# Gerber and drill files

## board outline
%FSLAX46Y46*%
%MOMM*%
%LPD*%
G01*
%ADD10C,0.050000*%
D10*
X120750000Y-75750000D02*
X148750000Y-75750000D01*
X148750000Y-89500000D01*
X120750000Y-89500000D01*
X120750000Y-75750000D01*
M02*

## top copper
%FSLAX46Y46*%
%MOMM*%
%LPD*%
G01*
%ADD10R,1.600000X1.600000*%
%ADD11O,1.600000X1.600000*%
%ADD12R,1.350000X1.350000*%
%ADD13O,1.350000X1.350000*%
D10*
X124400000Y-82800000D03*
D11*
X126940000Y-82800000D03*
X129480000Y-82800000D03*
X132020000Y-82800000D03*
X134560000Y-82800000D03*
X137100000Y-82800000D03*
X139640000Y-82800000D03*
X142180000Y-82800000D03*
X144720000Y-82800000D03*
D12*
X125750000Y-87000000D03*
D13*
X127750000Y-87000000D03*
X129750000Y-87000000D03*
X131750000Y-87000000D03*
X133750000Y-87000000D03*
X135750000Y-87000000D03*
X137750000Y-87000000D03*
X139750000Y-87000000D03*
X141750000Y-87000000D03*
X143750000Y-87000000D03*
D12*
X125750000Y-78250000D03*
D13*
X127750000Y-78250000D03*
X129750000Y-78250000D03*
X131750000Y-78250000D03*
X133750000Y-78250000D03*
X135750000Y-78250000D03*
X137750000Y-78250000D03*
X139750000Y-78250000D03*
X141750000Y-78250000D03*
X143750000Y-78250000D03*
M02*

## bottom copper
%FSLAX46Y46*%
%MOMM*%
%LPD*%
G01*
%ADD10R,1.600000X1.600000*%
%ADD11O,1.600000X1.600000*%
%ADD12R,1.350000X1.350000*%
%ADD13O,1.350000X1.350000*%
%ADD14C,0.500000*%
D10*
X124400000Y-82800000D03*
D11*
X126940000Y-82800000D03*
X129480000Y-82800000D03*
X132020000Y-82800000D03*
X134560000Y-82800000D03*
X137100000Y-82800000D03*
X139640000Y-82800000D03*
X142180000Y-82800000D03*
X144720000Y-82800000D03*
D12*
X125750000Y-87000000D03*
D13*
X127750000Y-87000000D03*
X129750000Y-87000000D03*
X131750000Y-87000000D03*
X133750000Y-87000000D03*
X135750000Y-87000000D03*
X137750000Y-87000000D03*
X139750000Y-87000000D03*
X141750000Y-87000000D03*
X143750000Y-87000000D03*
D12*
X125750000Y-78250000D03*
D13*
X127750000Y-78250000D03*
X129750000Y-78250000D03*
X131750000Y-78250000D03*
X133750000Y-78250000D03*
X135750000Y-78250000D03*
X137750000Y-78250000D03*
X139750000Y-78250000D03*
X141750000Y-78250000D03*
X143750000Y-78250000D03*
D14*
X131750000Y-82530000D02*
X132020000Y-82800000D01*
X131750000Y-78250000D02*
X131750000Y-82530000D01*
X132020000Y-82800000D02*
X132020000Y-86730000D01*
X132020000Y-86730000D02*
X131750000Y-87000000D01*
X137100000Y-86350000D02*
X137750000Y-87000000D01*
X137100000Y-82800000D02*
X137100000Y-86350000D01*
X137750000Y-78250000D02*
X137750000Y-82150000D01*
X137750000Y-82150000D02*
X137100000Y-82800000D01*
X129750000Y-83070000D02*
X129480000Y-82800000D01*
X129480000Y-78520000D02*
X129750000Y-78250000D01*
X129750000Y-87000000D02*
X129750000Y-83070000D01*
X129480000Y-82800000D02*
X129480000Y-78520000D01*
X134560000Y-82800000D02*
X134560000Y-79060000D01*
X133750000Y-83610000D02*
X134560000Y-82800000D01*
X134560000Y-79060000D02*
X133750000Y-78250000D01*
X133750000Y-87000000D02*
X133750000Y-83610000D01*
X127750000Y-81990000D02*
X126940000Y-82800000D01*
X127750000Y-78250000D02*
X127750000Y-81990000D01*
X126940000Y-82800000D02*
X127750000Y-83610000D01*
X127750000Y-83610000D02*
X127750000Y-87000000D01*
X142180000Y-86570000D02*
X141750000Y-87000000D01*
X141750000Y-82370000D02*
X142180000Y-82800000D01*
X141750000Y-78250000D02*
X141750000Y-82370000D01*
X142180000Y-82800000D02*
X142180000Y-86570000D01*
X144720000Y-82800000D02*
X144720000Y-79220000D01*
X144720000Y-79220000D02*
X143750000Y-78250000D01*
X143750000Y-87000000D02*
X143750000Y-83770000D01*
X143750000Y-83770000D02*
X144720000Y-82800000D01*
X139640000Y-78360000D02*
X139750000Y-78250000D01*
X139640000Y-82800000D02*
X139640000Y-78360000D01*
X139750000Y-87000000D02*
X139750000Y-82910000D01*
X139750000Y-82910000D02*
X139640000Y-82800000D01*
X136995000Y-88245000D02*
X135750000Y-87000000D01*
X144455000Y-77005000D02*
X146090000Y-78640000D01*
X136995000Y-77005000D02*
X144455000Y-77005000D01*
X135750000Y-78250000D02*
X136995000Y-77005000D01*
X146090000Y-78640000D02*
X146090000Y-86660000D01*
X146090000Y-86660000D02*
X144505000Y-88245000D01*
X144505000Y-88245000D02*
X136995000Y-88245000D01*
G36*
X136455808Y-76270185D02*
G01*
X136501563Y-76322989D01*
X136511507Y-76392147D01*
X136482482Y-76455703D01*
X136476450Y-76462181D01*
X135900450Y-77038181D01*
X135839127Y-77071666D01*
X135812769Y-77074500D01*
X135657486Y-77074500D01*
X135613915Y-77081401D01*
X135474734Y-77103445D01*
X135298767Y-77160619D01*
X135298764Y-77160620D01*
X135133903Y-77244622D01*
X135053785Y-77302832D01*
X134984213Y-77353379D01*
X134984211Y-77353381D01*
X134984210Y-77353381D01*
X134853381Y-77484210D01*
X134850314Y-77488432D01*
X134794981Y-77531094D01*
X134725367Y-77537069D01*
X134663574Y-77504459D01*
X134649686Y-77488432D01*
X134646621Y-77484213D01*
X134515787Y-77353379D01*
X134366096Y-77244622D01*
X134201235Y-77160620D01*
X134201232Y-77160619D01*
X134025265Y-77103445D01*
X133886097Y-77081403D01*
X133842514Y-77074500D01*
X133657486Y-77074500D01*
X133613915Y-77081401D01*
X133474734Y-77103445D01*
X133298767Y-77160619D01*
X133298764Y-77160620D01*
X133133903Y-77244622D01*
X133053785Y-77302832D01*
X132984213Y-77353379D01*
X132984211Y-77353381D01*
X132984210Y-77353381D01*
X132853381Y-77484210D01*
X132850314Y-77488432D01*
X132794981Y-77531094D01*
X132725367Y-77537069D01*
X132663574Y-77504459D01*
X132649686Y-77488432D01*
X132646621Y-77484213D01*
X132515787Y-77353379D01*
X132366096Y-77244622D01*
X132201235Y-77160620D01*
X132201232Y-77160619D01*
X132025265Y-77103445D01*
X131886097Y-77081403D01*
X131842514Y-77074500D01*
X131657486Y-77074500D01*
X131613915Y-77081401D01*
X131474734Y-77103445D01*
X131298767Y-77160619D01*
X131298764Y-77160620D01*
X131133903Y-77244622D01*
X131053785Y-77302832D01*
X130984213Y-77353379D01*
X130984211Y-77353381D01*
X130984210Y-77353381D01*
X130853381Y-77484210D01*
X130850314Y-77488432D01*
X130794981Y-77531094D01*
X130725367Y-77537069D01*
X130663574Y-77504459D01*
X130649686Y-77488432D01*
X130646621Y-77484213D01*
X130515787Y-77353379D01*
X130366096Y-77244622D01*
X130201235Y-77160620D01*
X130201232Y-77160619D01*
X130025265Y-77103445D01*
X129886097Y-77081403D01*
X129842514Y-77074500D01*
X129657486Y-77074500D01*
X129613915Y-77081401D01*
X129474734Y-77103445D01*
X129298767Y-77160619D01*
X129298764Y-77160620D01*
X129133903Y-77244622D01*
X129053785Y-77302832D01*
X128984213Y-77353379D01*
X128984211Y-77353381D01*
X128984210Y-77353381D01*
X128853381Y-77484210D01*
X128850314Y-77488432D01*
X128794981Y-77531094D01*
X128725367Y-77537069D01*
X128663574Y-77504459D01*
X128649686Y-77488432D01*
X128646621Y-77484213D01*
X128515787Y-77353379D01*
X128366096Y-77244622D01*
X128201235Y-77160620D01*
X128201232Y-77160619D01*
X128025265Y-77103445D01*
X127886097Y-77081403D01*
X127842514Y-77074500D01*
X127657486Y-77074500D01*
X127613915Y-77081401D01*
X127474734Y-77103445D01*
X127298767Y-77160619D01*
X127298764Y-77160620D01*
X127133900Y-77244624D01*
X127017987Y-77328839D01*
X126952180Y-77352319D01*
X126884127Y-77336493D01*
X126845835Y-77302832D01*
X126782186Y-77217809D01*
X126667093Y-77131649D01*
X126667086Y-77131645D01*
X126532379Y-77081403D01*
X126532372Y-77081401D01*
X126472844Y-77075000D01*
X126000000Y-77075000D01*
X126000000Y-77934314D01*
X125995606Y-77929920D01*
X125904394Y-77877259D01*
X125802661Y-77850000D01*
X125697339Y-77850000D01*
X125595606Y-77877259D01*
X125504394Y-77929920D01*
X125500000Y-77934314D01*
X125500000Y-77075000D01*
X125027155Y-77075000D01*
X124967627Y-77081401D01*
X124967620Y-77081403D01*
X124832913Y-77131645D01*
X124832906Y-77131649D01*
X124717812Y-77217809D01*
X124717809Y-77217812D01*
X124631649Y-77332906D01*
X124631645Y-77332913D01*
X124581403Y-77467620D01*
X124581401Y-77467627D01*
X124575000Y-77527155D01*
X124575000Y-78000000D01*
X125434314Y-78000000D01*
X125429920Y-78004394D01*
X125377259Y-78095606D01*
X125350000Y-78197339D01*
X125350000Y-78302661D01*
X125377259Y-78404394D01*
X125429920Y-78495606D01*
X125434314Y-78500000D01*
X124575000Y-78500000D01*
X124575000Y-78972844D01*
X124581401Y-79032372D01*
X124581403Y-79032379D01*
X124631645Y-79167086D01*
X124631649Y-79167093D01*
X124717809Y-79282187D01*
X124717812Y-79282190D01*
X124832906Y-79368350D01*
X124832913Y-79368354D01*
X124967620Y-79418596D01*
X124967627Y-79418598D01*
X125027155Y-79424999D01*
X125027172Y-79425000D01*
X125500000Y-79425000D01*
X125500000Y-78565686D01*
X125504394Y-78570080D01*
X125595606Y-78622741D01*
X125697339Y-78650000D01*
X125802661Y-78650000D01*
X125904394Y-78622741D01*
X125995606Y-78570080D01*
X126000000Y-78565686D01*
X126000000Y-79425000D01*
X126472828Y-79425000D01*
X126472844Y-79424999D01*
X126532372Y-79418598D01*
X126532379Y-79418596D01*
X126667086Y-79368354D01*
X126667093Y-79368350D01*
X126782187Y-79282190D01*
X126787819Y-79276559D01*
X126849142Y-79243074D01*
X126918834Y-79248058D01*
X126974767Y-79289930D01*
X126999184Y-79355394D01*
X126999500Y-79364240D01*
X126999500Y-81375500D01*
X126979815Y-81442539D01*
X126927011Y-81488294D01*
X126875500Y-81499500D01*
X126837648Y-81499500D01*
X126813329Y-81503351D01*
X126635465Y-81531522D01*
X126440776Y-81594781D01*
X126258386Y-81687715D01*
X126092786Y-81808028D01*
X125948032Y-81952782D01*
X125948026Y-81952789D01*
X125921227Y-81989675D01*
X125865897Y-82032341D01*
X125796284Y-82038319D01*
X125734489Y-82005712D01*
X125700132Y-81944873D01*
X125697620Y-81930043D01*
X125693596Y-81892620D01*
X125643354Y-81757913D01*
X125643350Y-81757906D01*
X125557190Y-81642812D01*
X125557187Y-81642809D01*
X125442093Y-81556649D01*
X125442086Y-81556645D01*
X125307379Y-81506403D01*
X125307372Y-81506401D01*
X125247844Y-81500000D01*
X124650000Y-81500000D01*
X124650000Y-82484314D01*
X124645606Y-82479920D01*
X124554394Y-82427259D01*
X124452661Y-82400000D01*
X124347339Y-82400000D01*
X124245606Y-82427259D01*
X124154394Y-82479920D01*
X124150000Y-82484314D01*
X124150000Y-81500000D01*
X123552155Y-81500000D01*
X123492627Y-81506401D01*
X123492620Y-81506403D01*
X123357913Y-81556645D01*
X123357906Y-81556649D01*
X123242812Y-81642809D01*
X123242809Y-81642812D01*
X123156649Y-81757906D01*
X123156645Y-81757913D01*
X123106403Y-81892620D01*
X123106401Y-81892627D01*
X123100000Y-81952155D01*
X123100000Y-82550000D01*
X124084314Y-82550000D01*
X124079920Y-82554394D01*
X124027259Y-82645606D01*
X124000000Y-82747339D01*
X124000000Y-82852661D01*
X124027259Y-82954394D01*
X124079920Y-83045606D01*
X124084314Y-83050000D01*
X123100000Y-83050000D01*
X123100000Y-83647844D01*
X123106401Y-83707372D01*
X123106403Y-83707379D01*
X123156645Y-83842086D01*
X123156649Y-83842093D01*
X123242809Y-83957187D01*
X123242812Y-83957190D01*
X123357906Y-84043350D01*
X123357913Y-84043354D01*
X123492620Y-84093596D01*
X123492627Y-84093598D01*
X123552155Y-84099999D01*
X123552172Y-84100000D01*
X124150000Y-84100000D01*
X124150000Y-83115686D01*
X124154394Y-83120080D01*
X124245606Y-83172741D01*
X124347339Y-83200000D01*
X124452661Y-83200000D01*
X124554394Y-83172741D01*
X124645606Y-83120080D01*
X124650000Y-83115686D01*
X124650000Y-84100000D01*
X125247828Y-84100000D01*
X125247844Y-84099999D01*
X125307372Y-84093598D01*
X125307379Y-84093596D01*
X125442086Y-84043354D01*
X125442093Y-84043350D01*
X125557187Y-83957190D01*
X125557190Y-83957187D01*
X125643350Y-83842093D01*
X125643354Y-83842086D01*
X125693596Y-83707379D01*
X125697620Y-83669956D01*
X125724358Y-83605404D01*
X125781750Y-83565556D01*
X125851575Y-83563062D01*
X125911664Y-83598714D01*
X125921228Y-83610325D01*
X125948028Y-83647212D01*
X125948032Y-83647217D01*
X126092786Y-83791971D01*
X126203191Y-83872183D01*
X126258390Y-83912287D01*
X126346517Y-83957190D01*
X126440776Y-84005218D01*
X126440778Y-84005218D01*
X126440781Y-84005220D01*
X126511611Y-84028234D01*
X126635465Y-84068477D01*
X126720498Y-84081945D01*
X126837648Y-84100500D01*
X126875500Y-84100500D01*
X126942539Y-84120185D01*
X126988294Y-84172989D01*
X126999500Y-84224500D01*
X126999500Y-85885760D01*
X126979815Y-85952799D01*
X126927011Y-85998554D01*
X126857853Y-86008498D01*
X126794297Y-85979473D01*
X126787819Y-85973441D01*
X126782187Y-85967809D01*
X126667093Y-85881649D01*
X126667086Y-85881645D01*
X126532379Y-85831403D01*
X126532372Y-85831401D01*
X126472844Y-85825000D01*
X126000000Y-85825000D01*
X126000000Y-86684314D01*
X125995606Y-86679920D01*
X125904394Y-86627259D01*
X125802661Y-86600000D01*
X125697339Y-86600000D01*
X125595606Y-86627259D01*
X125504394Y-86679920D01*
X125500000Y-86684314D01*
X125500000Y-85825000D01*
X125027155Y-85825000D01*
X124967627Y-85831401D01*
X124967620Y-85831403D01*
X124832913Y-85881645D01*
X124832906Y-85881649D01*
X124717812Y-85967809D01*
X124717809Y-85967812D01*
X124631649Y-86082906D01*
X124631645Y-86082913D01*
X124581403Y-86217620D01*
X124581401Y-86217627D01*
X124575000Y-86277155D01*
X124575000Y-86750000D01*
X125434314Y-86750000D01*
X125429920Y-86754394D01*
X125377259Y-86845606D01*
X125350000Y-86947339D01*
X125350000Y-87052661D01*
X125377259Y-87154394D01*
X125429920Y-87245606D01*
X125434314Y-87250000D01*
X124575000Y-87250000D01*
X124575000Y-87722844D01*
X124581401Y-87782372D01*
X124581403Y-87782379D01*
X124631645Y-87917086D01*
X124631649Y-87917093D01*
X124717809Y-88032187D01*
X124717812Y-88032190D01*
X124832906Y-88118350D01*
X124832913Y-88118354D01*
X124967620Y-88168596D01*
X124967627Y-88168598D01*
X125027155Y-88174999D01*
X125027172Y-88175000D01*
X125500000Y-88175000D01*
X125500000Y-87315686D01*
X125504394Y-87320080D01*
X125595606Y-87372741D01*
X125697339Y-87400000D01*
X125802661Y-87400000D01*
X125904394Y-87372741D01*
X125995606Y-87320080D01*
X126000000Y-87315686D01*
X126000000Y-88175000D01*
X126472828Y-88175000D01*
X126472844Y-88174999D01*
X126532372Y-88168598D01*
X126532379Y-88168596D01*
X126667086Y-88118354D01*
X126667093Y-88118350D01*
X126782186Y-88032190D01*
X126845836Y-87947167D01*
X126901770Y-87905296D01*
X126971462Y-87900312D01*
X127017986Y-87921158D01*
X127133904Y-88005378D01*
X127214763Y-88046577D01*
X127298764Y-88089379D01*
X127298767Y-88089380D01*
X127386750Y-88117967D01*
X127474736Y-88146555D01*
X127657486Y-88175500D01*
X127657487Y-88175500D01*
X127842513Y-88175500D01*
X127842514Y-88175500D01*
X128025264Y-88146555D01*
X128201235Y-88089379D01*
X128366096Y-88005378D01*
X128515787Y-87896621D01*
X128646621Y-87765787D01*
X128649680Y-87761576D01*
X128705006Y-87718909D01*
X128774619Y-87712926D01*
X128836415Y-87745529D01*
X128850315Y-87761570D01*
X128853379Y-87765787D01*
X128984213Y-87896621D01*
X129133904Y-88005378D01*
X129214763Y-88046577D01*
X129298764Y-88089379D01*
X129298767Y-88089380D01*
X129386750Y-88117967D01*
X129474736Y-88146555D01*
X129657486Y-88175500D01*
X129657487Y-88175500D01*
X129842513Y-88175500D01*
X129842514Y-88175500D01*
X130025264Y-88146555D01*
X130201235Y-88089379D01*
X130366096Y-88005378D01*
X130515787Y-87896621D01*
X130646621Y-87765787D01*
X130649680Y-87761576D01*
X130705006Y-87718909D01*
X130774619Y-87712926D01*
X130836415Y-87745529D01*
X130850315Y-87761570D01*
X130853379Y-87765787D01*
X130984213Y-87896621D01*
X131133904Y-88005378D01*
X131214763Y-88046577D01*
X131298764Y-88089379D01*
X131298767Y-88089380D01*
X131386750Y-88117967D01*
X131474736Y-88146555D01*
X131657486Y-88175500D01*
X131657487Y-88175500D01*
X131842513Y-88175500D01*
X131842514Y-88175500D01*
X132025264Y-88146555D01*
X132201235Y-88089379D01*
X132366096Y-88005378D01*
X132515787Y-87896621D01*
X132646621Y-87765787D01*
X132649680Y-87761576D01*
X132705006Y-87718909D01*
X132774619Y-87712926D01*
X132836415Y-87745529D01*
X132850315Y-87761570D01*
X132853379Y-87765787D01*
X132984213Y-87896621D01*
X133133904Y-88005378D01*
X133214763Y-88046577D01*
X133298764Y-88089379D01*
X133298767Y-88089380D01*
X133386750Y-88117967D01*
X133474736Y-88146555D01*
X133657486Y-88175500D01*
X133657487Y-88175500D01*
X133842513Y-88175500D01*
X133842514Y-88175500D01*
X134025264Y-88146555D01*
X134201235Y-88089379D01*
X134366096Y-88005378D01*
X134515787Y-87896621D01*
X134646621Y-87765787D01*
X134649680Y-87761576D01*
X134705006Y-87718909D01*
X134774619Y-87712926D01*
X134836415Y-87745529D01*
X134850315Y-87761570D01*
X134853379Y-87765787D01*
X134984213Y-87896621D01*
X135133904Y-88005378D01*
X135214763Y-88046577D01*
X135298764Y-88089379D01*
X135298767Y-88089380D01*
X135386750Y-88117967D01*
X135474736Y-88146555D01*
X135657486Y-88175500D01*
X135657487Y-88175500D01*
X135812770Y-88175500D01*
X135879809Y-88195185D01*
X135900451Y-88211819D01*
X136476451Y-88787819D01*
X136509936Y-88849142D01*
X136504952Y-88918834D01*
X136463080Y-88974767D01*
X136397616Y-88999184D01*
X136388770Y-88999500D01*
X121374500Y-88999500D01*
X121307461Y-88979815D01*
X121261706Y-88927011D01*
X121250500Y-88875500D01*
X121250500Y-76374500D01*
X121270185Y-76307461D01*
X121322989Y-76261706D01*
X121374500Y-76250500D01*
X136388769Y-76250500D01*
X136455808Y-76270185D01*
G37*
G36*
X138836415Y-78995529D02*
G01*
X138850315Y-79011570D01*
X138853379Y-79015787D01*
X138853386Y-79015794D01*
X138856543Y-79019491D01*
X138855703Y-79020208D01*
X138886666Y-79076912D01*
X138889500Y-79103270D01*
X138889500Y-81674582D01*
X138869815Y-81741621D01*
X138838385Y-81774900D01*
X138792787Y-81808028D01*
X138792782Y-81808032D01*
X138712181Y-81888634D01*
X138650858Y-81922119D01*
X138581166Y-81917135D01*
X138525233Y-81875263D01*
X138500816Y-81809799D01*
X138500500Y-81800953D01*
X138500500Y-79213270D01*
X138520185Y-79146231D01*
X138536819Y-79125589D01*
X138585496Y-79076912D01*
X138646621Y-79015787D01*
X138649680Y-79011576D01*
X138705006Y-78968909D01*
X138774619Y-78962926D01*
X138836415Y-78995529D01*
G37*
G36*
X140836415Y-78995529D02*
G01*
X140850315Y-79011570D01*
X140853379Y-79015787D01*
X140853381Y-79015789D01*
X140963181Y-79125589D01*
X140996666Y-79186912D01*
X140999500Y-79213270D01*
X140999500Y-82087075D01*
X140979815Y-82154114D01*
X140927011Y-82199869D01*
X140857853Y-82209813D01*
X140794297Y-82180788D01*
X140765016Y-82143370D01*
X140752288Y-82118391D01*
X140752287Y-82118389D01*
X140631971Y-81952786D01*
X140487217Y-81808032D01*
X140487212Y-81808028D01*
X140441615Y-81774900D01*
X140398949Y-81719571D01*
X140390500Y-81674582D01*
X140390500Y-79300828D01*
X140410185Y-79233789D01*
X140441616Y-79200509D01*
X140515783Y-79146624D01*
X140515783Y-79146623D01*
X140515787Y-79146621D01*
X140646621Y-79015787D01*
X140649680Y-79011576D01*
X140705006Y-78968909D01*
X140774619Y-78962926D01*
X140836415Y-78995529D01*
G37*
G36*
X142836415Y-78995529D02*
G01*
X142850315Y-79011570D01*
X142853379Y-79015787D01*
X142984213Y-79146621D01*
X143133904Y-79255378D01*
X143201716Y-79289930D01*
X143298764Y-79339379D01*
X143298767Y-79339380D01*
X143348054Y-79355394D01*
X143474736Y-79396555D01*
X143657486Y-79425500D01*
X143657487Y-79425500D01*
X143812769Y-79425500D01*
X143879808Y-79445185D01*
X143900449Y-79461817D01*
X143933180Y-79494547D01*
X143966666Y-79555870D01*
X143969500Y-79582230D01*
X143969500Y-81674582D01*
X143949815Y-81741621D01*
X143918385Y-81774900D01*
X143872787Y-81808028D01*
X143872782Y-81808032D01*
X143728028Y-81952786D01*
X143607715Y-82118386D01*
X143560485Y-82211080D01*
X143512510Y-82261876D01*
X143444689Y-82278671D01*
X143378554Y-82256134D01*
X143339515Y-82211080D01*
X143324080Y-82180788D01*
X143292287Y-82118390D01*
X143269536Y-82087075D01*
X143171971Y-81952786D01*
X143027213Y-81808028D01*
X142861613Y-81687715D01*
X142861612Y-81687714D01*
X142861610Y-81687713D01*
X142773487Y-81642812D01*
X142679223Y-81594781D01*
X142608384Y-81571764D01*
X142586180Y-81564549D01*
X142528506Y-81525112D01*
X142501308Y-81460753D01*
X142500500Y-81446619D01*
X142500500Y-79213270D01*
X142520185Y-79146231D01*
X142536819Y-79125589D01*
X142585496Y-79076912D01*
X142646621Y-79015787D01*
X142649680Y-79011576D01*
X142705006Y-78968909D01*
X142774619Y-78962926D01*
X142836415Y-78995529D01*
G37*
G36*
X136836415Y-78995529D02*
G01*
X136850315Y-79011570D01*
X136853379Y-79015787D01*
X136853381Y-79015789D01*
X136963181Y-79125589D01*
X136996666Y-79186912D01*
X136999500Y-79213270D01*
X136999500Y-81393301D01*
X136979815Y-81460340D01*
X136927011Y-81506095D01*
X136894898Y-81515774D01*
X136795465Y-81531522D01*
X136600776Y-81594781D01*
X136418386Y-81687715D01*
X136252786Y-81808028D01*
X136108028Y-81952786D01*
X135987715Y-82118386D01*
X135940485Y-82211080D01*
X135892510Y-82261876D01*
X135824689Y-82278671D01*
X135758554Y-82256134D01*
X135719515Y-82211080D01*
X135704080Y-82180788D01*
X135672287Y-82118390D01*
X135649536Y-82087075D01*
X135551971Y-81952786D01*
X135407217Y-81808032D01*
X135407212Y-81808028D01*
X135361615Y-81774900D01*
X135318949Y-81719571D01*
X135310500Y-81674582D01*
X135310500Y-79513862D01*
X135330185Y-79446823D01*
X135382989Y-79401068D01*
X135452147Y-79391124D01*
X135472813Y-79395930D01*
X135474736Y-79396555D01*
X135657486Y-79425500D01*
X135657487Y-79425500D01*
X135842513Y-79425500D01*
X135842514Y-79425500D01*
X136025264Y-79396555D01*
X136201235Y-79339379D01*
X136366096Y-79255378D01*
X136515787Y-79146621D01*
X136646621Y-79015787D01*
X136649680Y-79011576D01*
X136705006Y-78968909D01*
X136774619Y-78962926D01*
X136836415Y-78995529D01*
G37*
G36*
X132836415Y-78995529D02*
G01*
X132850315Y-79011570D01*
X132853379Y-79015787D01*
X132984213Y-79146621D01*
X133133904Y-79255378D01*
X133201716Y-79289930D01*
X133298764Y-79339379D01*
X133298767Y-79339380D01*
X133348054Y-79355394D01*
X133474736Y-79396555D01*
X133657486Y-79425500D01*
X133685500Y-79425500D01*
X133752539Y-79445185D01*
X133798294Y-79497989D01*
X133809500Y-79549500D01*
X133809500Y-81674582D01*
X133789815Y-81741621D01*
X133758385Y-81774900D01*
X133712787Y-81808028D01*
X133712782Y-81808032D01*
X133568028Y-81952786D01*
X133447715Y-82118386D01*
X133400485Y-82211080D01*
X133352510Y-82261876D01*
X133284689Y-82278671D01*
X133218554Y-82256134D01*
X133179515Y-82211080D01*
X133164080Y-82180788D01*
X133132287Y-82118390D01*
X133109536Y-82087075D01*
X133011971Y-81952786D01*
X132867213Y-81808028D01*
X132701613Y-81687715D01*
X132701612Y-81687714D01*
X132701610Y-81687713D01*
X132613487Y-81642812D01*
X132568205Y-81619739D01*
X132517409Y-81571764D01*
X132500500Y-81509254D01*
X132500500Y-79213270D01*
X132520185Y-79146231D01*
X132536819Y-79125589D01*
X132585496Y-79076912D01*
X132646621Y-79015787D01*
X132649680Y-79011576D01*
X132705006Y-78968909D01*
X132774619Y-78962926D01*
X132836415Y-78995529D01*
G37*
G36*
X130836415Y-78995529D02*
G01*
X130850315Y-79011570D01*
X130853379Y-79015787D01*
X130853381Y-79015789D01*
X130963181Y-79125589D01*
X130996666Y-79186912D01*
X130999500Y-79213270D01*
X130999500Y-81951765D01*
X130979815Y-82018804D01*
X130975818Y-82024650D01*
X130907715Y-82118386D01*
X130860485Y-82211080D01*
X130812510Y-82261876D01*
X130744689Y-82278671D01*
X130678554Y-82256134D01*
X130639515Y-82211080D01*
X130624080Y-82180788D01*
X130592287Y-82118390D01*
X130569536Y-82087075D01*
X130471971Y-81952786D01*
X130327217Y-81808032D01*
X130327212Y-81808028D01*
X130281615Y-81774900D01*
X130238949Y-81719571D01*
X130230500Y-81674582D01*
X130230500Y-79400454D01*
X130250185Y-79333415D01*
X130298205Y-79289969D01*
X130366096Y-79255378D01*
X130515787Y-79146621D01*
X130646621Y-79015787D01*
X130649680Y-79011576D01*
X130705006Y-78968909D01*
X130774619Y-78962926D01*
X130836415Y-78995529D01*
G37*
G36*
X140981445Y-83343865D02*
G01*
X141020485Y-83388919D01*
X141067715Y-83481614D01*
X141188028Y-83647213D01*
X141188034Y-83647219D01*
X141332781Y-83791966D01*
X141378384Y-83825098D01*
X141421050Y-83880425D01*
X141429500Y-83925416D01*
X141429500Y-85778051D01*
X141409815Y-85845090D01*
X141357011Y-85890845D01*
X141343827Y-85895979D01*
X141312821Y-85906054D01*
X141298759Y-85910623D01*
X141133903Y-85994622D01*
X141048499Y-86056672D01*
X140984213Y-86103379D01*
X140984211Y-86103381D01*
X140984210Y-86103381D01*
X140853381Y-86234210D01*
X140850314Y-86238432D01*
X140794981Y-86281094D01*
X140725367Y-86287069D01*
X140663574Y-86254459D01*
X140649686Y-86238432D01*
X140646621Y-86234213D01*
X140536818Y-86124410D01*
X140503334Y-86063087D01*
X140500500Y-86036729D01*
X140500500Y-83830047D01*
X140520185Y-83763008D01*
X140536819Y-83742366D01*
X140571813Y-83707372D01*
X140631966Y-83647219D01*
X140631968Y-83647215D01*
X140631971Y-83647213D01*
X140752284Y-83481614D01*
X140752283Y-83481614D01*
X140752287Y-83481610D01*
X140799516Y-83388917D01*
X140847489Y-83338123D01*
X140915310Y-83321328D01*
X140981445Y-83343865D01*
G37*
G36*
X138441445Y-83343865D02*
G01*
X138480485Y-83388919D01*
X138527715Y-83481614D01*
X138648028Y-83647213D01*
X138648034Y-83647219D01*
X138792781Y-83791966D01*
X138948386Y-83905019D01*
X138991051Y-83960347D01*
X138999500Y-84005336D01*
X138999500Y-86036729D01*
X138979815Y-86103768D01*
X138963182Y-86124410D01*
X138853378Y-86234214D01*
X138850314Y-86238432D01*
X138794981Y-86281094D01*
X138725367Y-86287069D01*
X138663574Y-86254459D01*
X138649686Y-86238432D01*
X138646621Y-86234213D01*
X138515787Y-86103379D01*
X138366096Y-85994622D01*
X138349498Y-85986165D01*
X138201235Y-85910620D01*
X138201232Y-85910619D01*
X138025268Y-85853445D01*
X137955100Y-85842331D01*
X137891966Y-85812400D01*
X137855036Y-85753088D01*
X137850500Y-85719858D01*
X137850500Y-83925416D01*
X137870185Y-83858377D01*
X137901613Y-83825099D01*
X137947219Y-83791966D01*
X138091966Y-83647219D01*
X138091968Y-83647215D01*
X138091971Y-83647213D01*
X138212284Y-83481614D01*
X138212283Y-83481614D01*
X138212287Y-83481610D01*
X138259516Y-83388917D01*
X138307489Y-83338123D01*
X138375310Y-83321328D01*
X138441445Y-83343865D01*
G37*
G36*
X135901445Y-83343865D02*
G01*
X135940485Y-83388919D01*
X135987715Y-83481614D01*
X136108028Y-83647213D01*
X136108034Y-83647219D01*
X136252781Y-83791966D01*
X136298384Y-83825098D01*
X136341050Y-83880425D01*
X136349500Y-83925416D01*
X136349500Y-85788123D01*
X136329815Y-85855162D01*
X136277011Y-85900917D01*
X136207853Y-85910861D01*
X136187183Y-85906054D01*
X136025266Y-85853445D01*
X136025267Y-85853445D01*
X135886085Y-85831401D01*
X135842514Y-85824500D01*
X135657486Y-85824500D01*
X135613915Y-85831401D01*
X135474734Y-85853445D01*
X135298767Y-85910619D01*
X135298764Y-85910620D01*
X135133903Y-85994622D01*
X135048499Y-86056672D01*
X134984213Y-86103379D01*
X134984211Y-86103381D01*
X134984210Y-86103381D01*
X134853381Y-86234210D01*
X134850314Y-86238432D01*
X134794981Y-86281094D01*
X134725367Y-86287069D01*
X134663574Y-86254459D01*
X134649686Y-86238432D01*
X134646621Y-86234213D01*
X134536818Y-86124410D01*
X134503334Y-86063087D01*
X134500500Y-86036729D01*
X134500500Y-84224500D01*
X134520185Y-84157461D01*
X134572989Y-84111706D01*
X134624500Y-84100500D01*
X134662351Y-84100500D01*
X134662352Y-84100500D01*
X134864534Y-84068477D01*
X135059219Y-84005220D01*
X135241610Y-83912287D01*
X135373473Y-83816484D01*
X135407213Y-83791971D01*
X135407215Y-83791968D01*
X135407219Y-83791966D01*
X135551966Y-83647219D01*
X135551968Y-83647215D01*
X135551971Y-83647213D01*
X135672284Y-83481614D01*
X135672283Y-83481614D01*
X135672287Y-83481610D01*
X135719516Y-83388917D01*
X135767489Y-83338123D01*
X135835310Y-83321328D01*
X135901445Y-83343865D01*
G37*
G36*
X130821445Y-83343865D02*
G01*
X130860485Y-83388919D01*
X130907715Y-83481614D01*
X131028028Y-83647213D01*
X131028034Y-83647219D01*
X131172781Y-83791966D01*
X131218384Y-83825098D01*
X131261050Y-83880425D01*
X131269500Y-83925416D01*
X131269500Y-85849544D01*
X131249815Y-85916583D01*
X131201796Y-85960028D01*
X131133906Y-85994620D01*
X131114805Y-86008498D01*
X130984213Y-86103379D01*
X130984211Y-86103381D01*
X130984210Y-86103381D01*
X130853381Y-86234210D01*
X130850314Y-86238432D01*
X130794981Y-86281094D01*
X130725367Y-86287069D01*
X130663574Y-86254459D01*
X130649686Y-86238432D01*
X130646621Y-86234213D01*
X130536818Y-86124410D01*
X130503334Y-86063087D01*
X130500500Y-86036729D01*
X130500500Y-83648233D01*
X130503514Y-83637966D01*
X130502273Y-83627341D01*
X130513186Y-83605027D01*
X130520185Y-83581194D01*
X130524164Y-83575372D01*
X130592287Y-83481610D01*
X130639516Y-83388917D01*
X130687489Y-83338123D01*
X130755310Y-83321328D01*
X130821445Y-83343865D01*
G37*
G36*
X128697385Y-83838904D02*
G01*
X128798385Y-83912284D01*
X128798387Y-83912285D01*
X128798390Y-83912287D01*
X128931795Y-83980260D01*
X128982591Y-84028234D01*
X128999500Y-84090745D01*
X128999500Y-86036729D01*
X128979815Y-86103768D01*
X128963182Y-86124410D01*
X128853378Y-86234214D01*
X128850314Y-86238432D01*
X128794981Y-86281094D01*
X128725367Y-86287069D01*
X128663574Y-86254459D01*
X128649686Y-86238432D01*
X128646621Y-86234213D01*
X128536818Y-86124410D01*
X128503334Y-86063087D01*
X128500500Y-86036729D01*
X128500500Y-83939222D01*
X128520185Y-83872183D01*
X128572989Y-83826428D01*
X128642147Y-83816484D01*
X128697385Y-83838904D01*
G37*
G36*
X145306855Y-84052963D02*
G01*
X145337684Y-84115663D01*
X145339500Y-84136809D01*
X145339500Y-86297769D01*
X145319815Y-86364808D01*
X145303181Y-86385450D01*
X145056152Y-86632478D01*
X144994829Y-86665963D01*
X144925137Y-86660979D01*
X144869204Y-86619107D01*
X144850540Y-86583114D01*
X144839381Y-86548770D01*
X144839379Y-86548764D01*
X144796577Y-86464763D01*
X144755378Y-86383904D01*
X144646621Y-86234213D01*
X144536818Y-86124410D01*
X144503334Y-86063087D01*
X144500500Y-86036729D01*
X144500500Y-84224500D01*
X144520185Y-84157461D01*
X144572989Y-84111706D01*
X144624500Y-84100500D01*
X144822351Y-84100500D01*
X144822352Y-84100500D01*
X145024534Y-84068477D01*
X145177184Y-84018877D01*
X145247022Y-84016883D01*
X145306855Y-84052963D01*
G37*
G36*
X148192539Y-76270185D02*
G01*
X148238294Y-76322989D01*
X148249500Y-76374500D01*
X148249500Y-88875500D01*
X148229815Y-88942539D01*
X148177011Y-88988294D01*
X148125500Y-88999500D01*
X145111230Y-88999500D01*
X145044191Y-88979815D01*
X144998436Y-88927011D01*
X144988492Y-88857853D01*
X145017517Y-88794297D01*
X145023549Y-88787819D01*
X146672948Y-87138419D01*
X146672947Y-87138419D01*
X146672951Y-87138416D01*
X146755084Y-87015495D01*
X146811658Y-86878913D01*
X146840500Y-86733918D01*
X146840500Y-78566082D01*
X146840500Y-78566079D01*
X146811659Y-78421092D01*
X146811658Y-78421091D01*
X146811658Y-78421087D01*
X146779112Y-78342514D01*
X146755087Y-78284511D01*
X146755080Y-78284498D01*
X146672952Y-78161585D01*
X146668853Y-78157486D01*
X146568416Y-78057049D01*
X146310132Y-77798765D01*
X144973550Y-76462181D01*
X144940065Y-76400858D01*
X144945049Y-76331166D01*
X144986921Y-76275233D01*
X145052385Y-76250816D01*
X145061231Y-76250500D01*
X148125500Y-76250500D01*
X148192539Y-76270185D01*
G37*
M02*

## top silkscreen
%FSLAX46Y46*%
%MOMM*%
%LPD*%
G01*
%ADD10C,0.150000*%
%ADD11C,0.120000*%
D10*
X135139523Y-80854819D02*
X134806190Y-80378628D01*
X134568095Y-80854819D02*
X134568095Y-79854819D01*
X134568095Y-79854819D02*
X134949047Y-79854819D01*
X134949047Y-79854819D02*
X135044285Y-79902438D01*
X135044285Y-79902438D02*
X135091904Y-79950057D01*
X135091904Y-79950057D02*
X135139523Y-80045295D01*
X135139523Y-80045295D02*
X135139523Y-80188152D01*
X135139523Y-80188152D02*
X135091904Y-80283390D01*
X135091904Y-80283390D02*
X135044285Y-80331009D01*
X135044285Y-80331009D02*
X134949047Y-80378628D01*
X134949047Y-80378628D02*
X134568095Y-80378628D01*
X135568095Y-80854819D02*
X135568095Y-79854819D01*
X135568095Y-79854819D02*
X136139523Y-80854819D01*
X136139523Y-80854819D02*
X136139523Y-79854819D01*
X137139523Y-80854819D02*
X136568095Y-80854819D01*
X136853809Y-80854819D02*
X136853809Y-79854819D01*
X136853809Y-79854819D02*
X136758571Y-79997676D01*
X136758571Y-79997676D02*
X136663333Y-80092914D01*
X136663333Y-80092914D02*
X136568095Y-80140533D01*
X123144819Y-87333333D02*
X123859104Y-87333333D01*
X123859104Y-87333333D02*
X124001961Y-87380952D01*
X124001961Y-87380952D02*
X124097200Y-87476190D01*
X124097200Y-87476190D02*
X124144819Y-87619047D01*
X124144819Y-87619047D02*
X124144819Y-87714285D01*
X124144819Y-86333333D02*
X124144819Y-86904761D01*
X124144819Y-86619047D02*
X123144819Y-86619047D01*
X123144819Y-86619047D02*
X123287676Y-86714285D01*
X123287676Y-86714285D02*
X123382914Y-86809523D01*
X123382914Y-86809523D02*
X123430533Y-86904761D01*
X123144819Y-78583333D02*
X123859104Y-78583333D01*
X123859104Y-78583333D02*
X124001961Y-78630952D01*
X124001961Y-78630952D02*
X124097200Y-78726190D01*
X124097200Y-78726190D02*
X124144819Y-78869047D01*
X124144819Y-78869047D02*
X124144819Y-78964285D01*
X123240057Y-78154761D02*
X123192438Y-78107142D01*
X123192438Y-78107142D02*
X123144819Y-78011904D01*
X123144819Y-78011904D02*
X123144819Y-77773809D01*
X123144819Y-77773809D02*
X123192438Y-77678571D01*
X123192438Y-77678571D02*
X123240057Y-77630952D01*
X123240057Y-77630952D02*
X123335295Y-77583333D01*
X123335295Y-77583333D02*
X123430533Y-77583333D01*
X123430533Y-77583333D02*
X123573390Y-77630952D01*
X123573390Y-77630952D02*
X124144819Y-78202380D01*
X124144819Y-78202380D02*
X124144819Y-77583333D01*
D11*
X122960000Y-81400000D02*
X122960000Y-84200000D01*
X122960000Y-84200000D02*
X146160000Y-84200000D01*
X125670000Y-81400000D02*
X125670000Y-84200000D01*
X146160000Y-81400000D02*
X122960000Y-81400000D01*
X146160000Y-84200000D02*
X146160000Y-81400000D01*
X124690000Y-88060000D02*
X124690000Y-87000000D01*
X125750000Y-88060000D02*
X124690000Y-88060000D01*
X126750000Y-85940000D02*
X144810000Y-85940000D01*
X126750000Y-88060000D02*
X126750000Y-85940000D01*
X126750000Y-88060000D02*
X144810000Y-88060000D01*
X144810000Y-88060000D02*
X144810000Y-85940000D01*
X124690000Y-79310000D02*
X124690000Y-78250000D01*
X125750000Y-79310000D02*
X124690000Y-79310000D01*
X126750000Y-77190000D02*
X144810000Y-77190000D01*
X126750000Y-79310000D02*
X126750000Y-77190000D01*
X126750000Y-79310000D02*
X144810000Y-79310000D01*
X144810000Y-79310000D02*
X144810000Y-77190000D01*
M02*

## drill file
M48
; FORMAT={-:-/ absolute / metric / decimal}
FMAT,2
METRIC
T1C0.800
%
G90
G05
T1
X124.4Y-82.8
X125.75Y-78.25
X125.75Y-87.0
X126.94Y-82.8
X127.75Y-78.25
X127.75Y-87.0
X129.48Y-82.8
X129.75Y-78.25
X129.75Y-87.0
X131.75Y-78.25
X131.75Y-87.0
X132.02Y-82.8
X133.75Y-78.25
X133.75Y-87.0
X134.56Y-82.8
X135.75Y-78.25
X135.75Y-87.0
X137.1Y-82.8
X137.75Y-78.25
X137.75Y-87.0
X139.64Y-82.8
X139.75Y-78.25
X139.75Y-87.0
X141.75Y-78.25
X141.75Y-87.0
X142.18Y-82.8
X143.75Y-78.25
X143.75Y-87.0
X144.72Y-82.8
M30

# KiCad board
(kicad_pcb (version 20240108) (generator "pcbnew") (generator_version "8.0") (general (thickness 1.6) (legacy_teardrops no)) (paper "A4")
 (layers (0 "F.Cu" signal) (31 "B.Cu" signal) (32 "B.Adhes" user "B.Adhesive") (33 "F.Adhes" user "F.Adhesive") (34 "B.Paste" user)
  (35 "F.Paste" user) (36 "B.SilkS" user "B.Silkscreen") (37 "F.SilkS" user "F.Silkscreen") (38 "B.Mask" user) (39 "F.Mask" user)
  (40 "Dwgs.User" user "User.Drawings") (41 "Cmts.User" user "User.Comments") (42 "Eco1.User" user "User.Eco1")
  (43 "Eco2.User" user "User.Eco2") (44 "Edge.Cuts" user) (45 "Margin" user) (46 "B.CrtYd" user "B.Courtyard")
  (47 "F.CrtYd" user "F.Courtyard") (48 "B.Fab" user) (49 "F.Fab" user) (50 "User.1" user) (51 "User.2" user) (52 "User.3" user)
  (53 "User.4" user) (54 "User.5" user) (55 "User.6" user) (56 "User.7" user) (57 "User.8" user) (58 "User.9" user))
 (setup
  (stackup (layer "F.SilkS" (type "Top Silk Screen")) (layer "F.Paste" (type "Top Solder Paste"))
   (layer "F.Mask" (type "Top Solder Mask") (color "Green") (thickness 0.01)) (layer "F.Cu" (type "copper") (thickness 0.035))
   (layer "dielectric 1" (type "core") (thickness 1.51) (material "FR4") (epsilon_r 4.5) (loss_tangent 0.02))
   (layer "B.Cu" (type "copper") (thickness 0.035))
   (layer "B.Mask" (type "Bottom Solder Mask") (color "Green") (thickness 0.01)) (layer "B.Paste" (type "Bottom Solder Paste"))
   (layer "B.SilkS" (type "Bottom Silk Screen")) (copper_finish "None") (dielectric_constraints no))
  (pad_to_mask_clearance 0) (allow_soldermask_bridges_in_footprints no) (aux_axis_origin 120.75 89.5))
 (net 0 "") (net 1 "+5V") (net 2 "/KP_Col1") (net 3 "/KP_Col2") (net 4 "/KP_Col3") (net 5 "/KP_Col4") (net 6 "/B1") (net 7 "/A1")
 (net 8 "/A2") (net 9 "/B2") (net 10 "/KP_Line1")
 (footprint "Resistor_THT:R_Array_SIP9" (layer "F.Cu") (at 124.4 82.8)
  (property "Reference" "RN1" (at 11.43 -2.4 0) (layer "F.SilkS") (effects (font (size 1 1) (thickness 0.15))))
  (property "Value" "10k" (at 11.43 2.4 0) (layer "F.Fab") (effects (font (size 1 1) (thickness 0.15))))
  (fp_line (start -1.44 -1.4) (end -1.44 1.4) (stroke (width 0.12) (type solid)) (layer "F.SilkS"))
  (fp_line (start -1.44 1.4) (end 21.76 1.4) (stroke (width 0.12) (type solid)) (layer "F.SilkS"))
  (fp_line (start 1.27 -1.4) (end 1.27 1.4) (stroke (width 0.12) (type solid)) (layer "F.SilkS"))
  (fp_line (start 21.76 -1.4) (end -1.44 -1.4) (stroke (width 0.12) (type solid)) (layer "F.SilkS"))
  (fp_line (start 21.76 1.4) (end 21.76 -1.4) (stroke (width 0.12) (type solid)) (layer "F.SilkS"))
  (pad "1" thru_hole rect (at 0 0) (size 1.6 1.6) (drill 0.8) (layers "*.Cu" "*.Mask") (remove_unused_layers no) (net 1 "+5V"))
  (pad "2" thru_hole oval (at 2.54 0) (size 1.6 1.6) (drill 0.8) (layers "*.Cu" "*.Mask") (remove_unused_layers no) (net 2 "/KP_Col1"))
  (pad "3" thru_hole oval (at 5.08 0) (size 1.6 1.6) (drill 0.8) (layers "*.Cu" "*.Mask") (remove_unused_layers no) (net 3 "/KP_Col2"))
  (pad "4" thru_hole oval (at 7.62 0) (size 1.6 1.6) (drill 0.8) (layers "*.Cu" "*.Mask") (remove_unused_layers no) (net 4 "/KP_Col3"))
  (pad "5" thru_hole oval (at 10.16 0) (size 1.6 1.6) (drill 0.8) (layers "*.Cu" "*.Mask") (remove_unused_layers no) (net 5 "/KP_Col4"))
  (pad "6" thru_hole oval (at 12.7 0) (size 1.6 1.6) (drill 0.8) (layers "*.Cu" "*.Mask") (remove_unused_layers no) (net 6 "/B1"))
  (pad "7" thru_hole oval (at 15.24 0) (size 1.6 1.6) (drill 0.8) (layers "*.Cu" "*.Mask") (remove_unused_layers no) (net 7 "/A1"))
  (pad "8" thru_hole oval (at 17.78 0) (size 1.6 1.6) (drill 0.8) (layers "*.Cu" "*.Mask") (remove_unused_layers no) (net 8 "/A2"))
  (pad "9" thru_hole oval (at 20.32 0) (size 1.6 1.6) (drill 0.8) (layers "*.Cu" "*.Mask") (remove_unused_layers no) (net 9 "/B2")))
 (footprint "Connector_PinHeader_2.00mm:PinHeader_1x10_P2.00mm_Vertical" (layer "F.Cu") (at 125.75 87 90)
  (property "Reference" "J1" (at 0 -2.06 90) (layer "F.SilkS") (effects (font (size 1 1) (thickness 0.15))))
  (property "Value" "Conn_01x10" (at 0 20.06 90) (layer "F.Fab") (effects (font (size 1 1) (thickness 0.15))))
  (fp_line (start -1.06 -1.06) (end 0 -1.06) (stroke (width 0.12) (type solid)) (layer "F.SilkS"))
  (fp_line (start -1.06 0) (end -1.06 -1.06) (stroke (width 0.12) (type solid)) (layer "F.SilkS"))
  (fp_line (start 1.06 1) (end 1.06 19.06) (stroke (width 0.12) (type solid)) (layer "F.SilkS"))
  (fp_line (start -1.06 1) (end 1.06 1) (stroke (width 0.12) (type solid)) (layer "F.SilkS"))
  (fp_line (start -1.06 1) (end -1.06 19.06) (stroke (width 0.12) (type solid)) (layer "F.SilkS"))
  (fp_line (start -1.06 19.06) (end 1.06 19.06) (stroke (width 0.12) (type solid)) (layer "F.SilkS"))
  (pad "1" thru_hole rect (at 0 0 90) (size 1.35 1.35) (drill 0.8) (layers "*.Cu" "*.Mask") (remove_unused_layers no) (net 1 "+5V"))
  (pad "2" thru_hole oval (at 0 2 90) (size 1.35 1.35) (drill 0.8) (layers "*.Cu" "*.Mask") (remove_unused_layers no) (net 2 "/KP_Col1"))
  (pad "3" thru_hole oval (at 0 4 90) (size 1.35 1.35) (drill 0.8) (layers "*.Cu" "*.Mask") (remove_unused_layers no) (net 3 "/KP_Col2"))
  (pad "4" thru_hole oval (at 0 6 90) (size 1.35 1.35) (drill 0.8) (layers "*.Cu" "*.Mask") (remove_unused_layers no) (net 4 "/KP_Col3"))
  (pad "5" thru_hole oval (at 0 8 90) (size 1.35 1.35) (drill 0.8) (layers "*.Cu" "*.Mask") (remove_unused_layers no) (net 5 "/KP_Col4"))
  (pad "6" thru_hole oval (at 0 10 90) (size 1.35 1.35) (drill 0.8) (layers "*.Cu" "*.Mask") (remove_unused_layers no) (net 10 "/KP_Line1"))
  (pad "7" thru_hole oval (at 0 12 90) (size 1.35 1.35) (drill 0.8) (layers "*.Cu" "*.Mask") (remove_unused_layers no) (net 6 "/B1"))
  (pad "8" thru_hole oval (at 0 14 90) (size 1.35 1.35) (drill 0.8) (layers "*.Cu" "*.Mask") (remove_unused_layers no) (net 7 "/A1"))
  (pad "9" thru_hole oval (at 0 16 90) (size 1.35 1.35) (drill 0.8) (layers "*.Cu" "*.Mask") (remove_unused_layers no) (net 8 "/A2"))
  (pad "10" thru_hole oval (at 0 18 90) (size 1.35 1.35) (drill 0.8) (layers "*.Cu" "*.Mask") (remove_unused_layers no) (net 9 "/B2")))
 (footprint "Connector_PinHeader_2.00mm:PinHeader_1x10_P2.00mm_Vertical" (layer "F.Cu") (at 125.75 78.25 90)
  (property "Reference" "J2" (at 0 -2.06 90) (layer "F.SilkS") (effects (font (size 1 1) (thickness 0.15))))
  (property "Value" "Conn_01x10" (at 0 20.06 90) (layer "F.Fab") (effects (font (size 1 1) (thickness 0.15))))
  (fp_line (start -1.06 -1.06) (end 0 -1.06) (stroke (width 0.12) (type solid)) (layer "F.SilkS"))
  (fp_line (start -1.06 0) (end -1.06 -1.06) (stroke (width 0.12) (type solid)) (layer "F.SilkS"))
  (fp_line (start 1.06 1) (end 1.06 19.06) (stroke (width 0.12) (type solid)) (layer "F.SilkS"))
  (fp_line (start -1.06 1) (end 1.06 1) (stroke (width 0.12) (type solid)) (layer "F.SilkS"))
  (fp_line (start -1.06 1) (end -1.06 19.06) (stroke (width 0.12) (type solid)) (layer "F.SilkS"))
  (fp_line (start -1.06 19.06) (end 1.06 19.06) (stroke (width 0.12) (type solid)) (layer "F.SilkS"))
  (pad "1" thru_hole rect (at 0 0 90) (size 1.35 1.35) (drill 0.8) (layers "*.Cu" "*.Mask") (remove_unused_layers no) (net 1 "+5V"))
  (pad "2" thru_hole oval (at 0 2 90) (size 1.35 1.35) (drill 0.8) (layers "*.Cu" "*.Mask") (remove_unused_layers no) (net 2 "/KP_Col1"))
  (pad "3" thru_hole oval (at 0 4 90) (size 1.35 1.35) (drill 0.8) (layers "*.Cu" "*.Mask") (remove_unused_layers no) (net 3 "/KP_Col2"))
  (pad "4" thru_hole oval (at 0 6 90) (size 1.35 1.35) (drill 0.8) (layers "*.Cu" "*.Mask") (remove_unused_layers no) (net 4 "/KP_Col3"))
  (pad "5" thru_hole oval (at 0 8 90) (size 1.35 1.35) (drill 0.8) (layers "*.Cu" "*.Mask") (remove_unused_layers no) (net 5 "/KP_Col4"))
  (pad "6" thru_hole oval (at 0 10 90) (size 1.35 1.35) (drill 0.8) (layers "*.Cu" "*.Mask") (remove_unused_layers no) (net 10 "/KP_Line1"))
  (pad "7" thru_hole oval (at 0 12 90) (size 1.35 1.35) (drill 0.8) (layers "*.Cu" "*.Mask") (remove_unused_layers no) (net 6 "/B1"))
  (pad "8" thru_hole oval (at 0 14 90) (size 1.35 1.35) (drill 0.8) (layers "*.Cu" "*.Mask") (remove_unused_layers no) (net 7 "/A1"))
  (pad "9" thru_hole oval (at 0 16 90) (size 1.35 1.35) (drill 0.8) (layers "*.Cu" "*.Mask") (remove_unused_layers no) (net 8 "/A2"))
  (pad "10" thru_hole oval (at 0 18 90) (size 1.35 1.35) (drill 0.8) (layers "*.Cu" "*.Mask") (remove_unused_layers no) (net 9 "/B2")))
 (gr_rect (start 120.75 75.75) (end 148.75 89.5) (stroke (width 0.05) (type default)) (fill none) (layer "Edge.Cuts"))
 (segment (start 131.75 82.53) (end 132.02 82.8) (width 0.5) (layer "B.Cu") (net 4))
 (segment (start 131.75 78.25) (end 131.75 82.53) (width 0.5) (layer "B.Cu") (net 4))
 (segment (start 132.02 82.8) (end 132.02 86.73) (width 0.5) (layer "B.Cu") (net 4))
 (segment (start 132.02 86.73) (end 131.75 87) (width 0.5) (layer "B.Cu") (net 4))
 (segment (start 137.1 86.35) (end 137.75 87) (width 0.5) (layer "B.Cu") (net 6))
 (segment (start 137.1 82.8) (end 137.1 86.35) (width 0.5) (layer "B.Cu") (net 6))
 (segment (start 137.75 78.25) (end 137.75 82.15) (width 0.5) (layer "B.Cu") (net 6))
 (segment (start 137.75 82.15) (end 137.1 82.8) (width 0.5) (layer "B.Cu") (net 6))
 (segment (start 129.75 83.07) (end 129.48 82.8) (width 0.5) (layer "B.Cu") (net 3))
 (segment (start 129.48 78.52) (end 129.75 78.25) (width 0.5) (layer "B.Cu") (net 3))
 (segment (start 129.75 87) (end 129.75 83.07) (width 0.5) (layer "B.Cu") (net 3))
 (segment (start 129.48 82.8) (end 129.48 78.52) (width 0.5) (layer "B.Cu") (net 3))
 (segment (start 134.56 82.8) (end 134.56 79.06) (width 0.5) (layer "B.Cu") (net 5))
 (segment (start 133.75 83.61) (end 134.56 82.8) (width 0.5) (layer "B.Cu") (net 5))
 (segment (start 134.56 79.06) (end 133.75 78.25) (width 0.5) (layer "B.Cu") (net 5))
 (segment (start 133.75 87) (end 133.75 83.61) (width 0.5) (layer "B.Cu") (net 5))
 (segment (start 127.75 81.99) (end 126.94 82.8) (width 0.5) (layer "B.Cu") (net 2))
 (segment (start 127.75 78.25) (end 127.75 81.99) (width 0.5) (layer "B.Cu") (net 2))
 (segment (start 126.94 82.8) (end 127.75 83.61) (width 0.5) (layer "B.Cu") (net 2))
 (segment (start 127.75 83.61) (end 127.75 87) (width 0.5) (layer "B.Cu") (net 2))
 (segment (start 142.18 86.57) (end 141.75 87) (width 0.5) (layer "B.Cu") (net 8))
 (segment (start 141.75 82.37) (end 142.18 82.8) (width 0.5) (layer "B.Cu") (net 8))
 (segment (start 141.75 78.25) (end 141.75 82.37) (width 0.5) (layer "B.Cu") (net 8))
 (segment (start 142.18 82.8) (end 142.18 86.57) (width 0.5) (layer "B.Cu") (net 8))
 (segment (start 144.72 82.8) (end 144.72 79.22) (width 0.5) (layer "B.Cu") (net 9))
 (segment (start 144.72 79.22) (end 143.75 78.25) (width 0.5) (layer "B.Cu") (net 9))
 (segment (start 143.75 87) (end 143.75 83.77) (width 0.5) (layer "B.Cu") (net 9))
 (segment (start 143.75 83.77) (end 144.72 82.8) (width 0.5) (layer "B.Cu") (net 9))
 (segment (start 139.64 78.36) (end 139.75 78.25) (width 0.5) (layer "B.Cu") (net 7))
 (segment (start 139.64 82.8) (end 139.64 78.36) (width 0.5) (layer "B.Cu") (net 7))
 (segment (start 139.75 87) (end 139.75 82.91) (width 0.5) (layer "B.Cu") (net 7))
 (segment (start 139.75 82.91) (end 139.64 82.8) (width 0.5) (layer "B.Cu") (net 7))
 (segment (start 136.995 88.245) (end 135.75 87) (width 0.5) (layer "B.Cu") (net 10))
 (segment (start 144.455 77.005) (end 146.09 78.64) (width 0.5) (layer "B.Cu") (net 10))
 (segment (start 136.995 77.005) (end 144.455 77.005) (width 0.5) (layer "B.Cu") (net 10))
 (segment (start 135.75 78.25) (end 136.995 77.005) (width 0.5) (layer "B.Cu") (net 10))
 (segment (start 146.09 78.64) (end 146.09 86.66) (width 0.5) (layer "B.Cu") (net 10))
 (segment (start 146.09 86.66) (end 144.505 88.245) (width 0.5) (layer "B.Cu") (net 10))
 (segment (start 144.505 88.245) (end 136.995 88.245) (width 0.5) (layer "B.Cu") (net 10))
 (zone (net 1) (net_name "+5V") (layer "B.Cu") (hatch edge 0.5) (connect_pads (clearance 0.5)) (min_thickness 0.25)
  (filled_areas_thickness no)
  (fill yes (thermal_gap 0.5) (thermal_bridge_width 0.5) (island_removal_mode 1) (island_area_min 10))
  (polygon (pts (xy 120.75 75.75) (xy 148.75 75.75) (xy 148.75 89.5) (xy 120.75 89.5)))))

